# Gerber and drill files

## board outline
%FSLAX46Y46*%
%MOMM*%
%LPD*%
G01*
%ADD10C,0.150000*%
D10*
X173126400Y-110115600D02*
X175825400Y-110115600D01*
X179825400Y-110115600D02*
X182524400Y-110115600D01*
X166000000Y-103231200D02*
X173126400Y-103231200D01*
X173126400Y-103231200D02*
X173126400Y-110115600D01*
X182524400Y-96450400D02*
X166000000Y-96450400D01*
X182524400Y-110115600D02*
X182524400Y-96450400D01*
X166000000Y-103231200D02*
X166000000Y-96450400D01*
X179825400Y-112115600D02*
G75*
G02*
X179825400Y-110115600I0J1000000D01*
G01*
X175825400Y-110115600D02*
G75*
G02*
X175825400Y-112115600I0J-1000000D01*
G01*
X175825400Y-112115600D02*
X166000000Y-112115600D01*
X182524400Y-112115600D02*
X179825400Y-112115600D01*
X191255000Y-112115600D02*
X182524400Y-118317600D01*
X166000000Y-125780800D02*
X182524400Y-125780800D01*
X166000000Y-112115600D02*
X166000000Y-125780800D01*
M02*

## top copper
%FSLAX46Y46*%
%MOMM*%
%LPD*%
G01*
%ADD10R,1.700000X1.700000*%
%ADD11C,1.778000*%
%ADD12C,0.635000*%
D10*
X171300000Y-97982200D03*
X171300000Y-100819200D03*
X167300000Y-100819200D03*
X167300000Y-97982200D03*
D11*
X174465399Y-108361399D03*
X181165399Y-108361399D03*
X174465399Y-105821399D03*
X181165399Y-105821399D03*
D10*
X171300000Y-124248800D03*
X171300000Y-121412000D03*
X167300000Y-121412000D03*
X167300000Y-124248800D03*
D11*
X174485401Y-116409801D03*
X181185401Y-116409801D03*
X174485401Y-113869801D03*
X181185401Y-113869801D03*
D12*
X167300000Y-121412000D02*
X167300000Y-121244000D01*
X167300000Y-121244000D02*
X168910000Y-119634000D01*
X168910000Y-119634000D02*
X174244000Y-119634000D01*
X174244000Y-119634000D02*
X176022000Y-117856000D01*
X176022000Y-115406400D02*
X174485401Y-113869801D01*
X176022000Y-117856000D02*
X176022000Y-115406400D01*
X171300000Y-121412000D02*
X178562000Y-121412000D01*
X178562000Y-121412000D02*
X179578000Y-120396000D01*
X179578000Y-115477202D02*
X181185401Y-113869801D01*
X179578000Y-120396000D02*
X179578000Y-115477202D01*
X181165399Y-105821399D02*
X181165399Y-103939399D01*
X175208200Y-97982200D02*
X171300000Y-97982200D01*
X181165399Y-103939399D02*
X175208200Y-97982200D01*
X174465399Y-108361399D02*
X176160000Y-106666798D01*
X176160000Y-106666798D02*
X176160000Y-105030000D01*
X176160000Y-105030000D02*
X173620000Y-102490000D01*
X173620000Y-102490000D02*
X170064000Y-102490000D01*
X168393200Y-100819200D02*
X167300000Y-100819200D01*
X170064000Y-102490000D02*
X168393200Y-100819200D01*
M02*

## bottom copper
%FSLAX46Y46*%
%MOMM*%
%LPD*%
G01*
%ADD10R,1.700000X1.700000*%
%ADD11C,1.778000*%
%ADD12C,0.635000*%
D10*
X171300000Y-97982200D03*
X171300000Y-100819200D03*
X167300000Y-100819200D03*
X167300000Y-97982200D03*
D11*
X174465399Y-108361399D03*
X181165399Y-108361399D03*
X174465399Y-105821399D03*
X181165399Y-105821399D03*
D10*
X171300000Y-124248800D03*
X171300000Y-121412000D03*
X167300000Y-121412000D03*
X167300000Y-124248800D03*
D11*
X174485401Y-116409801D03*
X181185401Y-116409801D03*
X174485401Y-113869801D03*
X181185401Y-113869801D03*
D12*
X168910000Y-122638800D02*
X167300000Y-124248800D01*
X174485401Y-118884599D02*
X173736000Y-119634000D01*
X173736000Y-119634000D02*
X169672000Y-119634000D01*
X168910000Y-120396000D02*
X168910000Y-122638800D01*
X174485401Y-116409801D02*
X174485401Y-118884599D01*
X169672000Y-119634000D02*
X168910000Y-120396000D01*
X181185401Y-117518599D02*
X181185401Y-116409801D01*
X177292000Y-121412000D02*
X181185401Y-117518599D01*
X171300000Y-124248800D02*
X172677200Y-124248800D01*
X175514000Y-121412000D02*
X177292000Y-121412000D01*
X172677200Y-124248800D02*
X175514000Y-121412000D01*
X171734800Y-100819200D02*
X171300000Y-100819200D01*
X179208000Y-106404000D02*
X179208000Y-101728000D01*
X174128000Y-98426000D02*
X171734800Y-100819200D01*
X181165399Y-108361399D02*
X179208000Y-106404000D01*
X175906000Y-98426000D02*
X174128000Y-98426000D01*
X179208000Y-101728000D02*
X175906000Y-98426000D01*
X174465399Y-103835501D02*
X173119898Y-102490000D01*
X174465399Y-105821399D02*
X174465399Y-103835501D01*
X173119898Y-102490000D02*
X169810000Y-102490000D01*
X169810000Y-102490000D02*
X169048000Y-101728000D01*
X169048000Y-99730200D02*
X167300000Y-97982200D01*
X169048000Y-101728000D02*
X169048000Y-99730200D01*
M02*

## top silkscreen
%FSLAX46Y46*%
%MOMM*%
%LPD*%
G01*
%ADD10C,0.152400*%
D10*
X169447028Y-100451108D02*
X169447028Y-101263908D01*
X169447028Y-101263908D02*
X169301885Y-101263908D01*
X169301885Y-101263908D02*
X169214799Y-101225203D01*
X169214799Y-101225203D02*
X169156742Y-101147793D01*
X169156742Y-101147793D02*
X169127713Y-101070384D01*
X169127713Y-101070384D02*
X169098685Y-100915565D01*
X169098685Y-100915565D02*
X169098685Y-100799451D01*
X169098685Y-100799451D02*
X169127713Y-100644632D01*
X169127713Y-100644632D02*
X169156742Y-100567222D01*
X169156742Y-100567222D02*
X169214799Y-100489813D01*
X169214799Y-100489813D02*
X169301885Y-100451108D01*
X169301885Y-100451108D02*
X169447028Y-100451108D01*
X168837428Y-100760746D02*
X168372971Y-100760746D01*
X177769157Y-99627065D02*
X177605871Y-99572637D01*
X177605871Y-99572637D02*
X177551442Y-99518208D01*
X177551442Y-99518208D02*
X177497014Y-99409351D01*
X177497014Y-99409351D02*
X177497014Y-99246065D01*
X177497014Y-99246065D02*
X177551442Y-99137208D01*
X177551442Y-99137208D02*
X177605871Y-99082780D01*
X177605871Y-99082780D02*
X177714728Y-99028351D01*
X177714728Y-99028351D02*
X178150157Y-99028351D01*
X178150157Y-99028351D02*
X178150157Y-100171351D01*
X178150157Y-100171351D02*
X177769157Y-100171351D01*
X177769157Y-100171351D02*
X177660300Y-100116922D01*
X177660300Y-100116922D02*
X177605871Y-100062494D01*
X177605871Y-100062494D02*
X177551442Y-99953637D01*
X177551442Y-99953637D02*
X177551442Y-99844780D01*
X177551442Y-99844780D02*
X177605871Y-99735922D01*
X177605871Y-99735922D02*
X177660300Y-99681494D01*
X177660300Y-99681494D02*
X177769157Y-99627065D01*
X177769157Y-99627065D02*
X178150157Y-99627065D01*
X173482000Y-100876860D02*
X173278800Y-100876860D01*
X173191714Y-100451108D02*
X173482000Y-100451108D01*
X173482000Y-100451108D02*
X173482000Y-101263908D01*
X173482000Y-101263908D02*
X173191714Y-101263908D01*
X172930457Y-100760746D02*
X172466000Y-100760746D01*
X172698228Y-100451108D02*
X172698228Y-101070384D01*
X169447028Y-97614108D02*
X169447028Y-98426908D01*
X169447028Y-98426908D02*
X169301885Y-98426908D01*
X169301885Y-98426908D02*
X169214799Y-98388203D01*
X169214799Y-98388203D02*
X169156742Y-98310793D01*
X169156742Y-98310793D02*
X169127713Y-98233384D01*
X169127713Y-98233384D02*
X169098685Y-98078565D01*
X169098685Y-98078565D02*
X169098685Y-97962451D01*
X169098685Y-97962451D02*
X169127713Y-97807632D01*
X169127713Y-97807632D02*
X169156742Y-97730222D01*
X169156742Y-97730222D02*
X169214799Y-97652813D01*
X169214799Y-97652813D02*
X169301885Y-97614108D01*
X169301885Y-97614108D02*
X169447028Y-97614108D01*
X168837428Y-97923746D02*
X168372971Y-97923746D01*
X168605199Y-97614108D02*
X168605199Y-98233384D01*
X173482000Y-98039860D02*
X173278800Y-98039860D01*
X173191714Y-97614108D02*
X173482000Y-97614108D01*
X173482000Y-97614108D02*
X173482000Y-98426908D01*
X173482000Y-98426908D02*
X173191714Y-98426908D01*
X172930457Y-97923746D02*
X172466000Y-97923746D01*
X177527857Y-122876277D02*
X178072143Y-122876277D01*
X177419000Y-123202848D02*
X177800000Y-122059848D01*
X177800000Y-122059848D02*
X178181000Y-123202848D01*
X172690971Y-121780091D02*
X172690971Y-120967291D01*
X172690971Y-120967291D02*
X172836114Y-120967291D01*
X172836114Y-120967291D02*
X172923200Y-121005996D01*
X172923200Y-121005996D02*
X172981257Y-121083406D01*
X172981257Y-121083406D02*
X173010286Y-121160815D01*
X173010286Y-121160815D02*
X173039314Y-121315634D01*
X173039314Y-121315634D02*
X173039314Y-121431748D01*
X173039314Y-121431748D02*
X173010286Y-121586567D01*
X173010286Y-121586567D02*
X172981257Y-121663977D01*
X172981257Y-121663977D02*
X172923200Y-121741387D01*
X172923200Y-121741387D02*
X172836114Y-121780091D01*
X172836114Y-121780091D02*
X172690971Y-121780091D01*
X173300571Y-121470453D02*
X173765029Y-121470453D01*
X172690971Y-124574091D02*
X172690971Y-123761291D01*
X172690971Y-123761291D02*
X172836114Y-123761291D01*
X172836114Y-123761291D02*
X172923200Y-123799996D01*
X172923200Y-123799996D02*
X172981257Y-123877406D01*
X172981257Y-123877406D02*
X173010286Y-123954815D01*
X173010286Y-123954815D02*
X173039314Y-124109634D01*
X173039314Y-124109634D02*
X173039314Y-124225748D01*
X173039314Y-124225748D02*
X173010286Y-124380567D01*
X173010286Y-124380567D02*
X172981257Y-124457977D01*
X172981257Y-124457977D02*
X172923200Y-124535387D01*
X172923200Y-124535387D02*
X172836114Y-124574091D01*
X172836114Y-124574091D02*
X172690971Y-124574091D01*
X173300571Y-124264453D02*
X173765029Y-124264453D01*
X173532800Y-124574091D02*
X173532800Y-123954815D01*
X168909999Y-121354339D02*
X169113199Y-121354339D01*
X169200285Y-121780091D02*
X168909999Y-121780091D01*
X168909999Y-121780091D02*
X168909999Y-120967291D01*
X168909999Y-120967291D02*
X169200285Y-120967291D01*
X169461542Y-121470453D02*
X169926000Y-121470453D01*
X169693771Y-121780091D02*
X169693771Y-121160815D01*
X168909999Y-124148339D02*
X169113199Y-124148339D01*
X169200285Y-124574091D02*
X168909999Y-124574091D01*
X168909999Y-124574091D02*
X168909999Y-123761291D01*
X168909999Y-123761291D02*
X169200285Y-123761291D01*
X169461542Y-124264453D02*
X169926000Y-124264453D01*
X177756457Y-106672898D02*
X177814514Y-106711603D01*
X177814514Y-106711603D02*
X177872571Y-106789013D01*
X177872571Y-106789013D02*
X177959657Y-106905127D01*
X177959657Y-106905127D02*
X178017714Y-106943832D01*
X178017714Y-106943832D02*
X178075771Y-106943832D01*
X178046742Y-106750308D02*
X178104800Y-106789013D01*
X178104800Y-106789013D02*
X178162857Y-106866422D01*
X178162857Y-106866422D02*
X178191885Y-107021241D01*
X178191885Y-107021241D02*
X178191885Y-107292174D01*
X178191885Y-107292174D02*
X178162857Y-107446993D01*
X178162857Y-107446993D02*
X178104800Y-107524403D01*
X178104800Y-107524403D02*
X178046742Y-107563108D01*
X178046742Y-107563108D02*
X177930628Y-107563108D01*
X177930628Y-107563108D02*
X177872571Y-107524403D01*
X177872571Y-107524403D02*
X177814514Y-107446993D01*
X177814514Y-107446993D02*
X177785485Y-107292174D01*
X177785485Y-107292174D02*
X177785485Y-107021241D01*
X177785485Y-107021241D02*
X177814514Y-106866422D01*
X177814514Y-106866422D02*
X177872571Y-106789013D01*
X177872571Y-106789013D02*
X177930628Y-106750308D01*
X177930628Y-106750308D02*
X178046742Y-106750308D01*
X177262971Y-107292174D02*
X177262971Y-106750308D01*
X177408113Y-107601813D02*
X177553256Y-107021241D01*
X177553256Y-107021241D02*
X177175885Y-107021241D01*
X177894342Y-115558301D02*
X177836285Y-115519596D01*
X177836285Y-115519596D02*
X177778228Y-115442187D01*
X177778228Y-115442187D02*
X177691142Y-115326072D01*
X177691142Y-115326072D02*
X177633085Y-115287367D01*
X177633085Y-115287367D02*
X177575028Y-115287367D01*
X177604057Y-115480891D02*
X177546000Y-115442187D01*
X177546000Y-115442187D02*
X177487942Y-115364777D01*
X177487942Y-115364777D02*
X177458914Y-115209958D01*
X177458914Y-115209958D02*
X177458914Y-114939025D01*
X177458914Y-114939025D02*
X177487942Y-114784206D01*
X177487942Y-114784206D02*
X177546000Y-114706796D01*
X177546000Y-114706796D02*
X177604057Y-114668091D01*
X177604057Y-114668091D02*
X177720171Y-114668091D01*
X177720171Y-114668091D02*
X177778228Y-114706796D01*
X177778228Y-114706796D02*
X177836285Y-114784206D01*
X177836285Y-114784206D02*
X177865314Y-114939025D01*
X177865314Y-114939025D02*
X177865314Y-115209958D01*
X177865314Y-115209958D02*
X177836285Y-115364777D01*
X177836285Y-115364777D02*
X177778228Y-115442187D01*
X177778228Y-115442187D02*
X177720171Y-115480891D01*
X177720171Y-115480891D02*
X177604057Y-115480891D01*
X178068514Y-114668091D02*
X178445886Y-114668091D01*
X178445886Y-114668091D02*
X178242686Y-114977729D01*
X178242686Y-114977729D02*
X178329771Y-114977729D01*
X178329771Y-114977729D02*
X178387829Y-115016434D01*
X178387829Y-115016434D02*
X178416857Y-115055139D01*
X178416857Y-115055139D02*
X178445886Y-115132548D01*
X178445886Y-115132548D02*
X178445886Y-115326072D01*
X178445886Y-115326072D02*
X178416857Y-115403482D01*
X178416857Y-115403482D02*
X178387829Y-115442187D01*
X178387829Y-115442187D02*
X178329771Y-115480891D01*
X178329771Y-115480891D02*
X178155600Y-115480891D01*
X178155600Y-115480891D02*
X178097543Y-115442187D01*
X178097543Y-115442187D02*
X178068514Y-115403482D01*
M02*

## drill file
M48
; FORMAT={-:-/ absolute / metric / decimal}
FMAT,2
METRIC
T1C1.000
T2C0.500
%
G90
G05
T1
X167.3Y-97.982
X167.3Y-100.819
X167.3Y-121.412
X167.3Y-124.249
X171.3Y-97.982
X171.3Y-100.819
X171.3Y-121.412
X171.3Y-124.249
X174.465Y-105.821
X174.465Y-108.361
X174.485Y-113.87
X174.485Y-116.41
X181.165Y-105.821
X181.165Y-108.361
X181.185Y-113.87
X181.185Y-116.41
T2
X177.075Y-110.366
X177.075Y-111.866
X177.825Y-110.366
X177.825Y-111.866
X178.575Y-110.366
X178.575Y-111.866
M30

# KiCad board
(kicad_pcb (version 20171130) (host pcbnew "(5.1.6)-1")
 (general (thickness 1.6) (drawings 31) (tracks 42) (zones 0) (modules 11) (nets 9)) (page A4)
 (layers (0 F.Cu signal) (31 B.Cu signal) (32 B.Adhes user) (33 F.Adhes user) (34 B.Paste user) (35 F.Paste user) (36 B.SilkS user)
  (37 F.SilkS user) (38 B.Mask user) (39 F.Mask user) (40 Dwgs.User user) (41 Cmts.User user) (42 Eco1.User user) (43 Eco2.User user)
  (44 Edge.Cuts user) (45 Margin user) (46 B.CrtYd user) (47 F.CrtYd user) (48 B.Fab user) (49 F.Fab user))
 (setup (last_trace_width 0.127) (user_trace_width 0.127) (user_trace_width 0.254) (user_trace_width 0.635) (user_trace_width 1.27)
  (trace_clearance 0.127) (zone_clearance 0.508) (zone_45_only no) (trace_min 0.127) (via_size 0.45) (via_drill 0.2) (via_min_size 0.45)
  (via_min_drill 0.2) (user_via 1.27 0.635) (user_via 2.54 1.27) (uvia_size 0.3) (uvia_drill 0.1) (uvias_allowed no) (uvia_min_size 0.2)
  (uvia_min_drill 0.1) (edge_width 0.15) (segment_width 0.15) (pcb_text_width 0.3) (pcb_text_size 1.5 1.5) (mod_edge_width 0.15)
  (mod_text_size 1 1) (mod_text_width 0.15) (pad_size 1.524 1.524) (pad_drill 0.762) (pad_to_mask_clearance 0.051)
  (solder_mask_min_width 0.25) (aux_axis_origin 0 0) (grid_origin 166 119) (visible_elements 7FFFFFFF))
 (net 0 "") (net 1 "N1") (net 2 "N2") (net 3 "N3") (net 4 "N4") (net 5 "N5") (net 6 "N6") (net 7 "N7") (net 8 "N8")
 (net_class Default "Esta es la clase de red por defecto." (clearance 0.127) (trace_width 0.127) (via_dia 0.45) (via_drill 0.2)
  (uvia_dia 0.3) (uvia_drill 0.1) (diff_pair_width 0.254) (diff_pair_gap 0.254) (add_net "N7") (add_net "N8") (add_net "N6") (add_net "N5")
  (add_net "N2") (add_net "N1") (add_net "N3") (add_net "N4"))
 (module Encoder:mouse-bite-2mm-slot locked (layer F.Cu) (at 177.8254 111.1156)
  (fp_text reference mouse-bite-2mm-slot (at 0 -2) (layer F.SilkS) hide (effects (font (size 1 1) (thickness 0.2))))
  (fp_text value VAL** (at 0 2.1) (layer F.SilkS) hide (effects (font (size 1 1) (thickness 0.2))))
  (pad "" np_thru_hole circle (at 0.75 0.75) (size 0.5 0.5) (drill 0.5) (layers *.Cu *.Mask))
  (pad "" np_thru_hole circle (at -0.75 0.75) (size 0.5 0.5) (drill 0.5) (layers *.Cu *.Mask))
  (pad "" np_thru_hole circle (at -0.75 -0.75) (size 0.5 0.5) (drill 0.5) (layers *.Cu *.Mask))
  (pad "" np_thru_hole circle (at 0.75 -0.75) (size 0.5 0.5) (drill 0.5) (layers *.Cu *.Mask))
  (pad "" np_thru_hole circle (at 0 0.75) (size 0.5 0.5) (drill 0.5) (layers *.Cu *.Mask))
  (pad "" np_thru_hole circle (at 0 -0.75) (size 0.5 0.5) (drill 0.5) (layers *.Cu *.Mask)))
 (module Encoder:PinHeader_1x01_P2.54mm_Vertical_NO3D (layer F.Cu) (at 171.3 97.9822 180)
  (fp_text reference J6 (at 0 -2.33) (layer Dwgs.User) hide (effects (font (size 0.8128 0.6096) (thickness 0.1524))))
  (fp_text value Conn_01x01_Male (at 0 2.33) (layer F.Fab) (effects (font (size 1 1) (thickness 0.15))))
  (pad 1 thru_hole rect (at 0 0 180) (size 1.7 1.7) (drill 1) (layers *.Cu *.Mask) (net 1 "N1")))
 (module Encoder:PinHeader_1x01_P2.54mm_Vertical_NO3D (layer F.Cu) (at 171.3 100.8192 180)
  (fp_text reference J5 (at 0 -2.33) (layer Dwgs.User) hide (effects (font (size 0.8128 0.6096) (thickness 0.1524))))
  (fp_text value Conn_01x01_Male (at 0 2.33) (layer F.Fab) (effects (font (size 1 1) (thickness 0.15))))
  (pad 1 thru_hole rect (at 0 0 180) (size 1.7 1.7) (drill 1) (layers *.Cu *.Mask) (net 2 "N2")))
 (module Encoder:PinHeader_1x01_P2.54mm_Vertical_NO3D (layer F.Cu) (at 167.3 100.8192 180)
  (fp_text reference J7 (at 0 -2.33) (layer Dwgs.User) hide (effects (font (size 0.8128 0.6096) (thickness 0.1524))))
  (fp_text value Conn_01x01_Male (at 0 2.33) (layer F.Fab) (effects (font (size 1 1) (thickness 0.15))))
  (pad 1 thru_hole rect (at 0 0 180) (size 1.7 1.7) (drill 1) (layers *.Cu *.Mask) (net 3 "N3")))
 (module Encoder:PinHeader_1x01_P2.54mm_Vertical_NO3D (layer F.Cu) (at 167.3 97.9822 180)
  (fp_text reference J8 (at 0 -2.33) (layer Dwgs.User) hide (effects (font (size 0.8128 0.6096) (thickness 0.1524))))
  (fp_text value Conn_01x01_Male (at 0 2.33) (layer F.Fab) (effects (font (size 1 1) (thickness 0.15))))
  (pad 1 thru_hole rect (at 0 0 180) (size 1.7 1.7) (drill 1) (layers *.Cu *.Mask) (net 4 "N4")))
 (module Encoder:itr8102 (layer F.Cu) (at 177.815399 107.091399 180)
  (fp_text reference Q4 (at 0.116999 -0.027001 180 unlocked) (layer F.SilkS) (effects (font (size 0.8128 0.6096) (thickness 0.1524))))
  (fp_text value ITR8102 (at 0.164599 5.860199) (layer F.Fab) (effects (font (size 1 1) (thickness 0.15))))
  (pad 4 thru_hole circle (at 3.35 -1.27 180) (size 1.778 1.778) (drill 1) (layers *.Cu *.Mask) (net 3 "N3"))
  (pad 1 thru_hole circle (at -3.35 -1.27 180) (size 1.778 1.778) (drill 1) (layers *.Cu *.Mask) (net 2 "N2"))
  (pad 3 thru_hole circle (at 3.35 1.27 180) (size 1.778 1.778) (drill 1) (layers *.Cu *.Mask) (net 4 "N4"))
  (pad 2 thru_hole circle (at -3.35 1.27 180) (size 1.778 1.778) (drill 1) (layers *.Cu *.Mask) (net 1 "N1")))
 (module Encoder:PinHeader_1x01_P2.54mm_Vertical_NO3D (layer F.Cu) (at 171.3 124.2488)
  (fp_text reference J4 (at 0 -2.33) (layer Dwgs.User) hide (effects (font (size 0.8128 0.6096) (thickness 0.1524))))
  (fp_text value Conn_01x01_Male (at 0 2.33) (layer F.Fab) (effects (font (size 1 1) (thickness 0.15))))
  (pad 1 thru_hole rect (at 0 0) (size 1.7 1.7) (drill 1) (layers *.Cu *.Mask) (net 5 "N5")))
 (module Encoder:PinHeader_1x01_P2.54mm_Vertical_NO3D (layer F.Cu) (at 171.3 121.412)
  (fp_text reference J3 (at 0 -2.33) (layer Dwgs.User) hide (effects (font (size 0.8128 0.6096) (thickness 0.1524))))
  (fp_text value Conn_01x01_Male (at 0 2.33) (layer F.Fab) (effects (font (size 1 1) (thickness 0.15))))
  (pad 1 thru_hole rect (at 0 0) (size 1.7 1.7) (drill 1) (layers *.Cu *.Mask) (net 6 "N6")))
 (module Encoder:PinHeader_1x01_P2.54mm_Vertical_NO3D (layer F.Cu) (at 167.3 121.412)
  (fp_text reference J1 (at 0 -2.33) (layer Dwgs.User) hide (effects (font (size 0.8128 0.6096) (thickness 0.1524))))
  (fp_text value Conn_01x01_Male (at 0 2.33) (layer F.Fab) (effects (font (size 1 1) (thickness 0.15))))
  (pad 1 thru_hole rect (at 0 0) (size 1.7 1.7) (drill 1) (layers *.Cu *.Mask) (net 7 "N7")))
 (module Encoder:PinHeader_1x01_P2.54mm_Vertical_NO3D (layer F.Cu) (at 167.3 124.2488)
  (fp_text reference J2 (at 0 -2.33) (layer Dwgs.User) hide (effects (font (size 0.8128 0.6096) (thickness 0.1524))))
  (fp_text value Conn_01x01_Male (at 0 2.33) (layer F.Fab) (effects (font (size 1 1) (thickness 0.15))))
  (pad 1 thru_hole rect (at 0 0) (size 1.7 1.7) (drill 1) (layers *.Cu *.Mask) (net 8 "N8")))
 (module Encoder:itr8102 (layer F.Cu) (at 177.835401 115.139801)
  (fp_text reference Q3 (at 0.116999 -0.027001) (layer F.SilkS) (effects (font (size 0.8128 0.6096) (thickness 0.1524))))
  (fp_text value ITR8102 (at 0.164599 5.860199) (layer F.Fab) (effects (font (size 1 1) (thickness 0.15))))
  (pad 2 thru_hole circle (at -3.35 1.27) (size 1.778 1.778) (drill 1) (layers *.Cu *.Mask) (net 8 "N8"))
  (pad 3 thru_hole circle (at 3.35 1.27) (size 1.778 1.778) (drill 1) (layers *.Cu *.Mask) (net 5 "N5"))
  (pad 1 thru_hole circle (at -3.35 -1.27) (size 1.778 1.778) (drill 1) (layers *.Cu *.Mask) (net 7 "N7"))
  (pad 4 thru_hole circle (at 3.35 -1.27) (size 1.778 1.778) (drill 1) (layers *.Cu *.Mask) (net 6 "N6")))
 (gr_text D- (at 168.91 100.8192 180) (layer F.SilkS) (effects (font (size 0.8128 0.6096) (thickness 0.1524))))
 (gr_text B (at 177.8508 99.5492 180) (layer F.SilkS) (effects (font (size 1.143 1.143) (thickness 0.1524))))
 (gr_line (start 173.1264 110.1156) (end 175.8254 110.1156) (layer Edge.Cuts) (width 0.15))
 (gr_line (start 179.8254 110.1156) (end 182.5244 110.1156) (layer Edge.Cuts) (width 0.15))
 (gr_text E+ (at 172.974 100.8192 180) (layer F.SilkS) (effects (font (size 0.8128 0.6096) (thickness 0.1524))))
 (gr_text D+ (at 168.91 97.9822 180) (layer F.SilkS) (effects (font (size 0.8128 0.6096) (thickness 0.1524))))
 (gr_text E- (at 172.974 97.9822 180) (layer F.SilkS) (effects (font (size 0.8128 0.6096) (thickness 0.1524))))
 (gr_line (start 166 103.2312) (end 173.1264 103.2312) (layer Edge.Cuts) (width 0.15))
 (gr_line (start 173.1264 103.2312) (end 173.1264 110.1156) (layer Edge.Cuts) (width 0.15))
 (gr_line (start 182.5244 96.4504) (end 166 96.4504) (layer Edge.Cuts) (width 0.15))
 (gr_line (start 182.5244 110.1156) (end 182.5244 96.4504) (layer Edge.Cuts) (width 0.15))
 (gr_line (start 166 103.2312) (end 166 96.4504) (layer Edge.Cuts) (width 0.15))
 (gr_arc (start 179.8254 111.1156) (end 179.8254 110.1156) (angle -180) (layer Edge.Cuts) (width 0.15))
 (gr_arc (start 175.8254 111.1156) (end 175.8254 112.1156) (angle -180) (layer Edge.Cuts) (width 0.15))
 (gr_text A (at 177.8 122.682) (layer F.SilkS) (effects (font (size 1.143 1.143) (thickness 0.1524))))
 (gr_line (start 175.8254 112.1156) (end 166 112.1156) (layer Edge.Cuts) (width 0.15))
 (gr_line (start 182.5244 112.1156) (end 179.8254 112.1156) (layer Edge.Cuts) (width 0.15))
 (gr_line (start 191.255 112.1156) (end 182.5244 118.3176) (layer Edge.Cuts) (width 0.15))
 (gr_line (start 166 125.7808) (end 182.5244 125.7808) (layer Edge.Cuts) (width 0.15))
 (gr_line (start 166 112.1156) (end 166 125.7808) (layer Edge.Cuts) (width 0.15))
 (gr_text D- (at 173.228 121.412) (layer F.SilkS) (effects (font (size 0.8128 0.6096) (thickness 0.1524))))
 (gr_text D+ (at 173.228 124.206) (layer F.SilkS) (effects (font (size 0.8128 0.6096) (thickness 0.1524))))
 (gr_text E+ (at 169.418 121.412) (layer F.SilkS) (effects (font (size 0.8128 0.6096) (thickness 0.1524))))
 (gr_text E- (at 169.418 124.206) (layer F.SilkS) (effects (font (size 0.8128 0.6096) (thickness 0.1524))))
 (segment (start 167.3 121.412) (end 167.3 121.244) (width 0.635) (layer F.Cu) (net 7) (status 30))
 (segment (start 167.3 121.244) (end 168.91 119.634) (width 0.635) (layer F.Cu) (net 7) (status 10))
 (segment (start 168.91 119.634) (end 174.244 119.634) (width 0.635) (layer F.Cu) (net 7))
 (segment (start 174.244 119.634) (end 176.022 117.856) (width 0.635) (layer F.Cu) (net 7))
 (segment (start 176.022 115.4064) (end 174.485401 113.869801) (width 0.635) (layer F.Cu) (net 7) (status 20))
 (segment (start 176.022 117.856) (end 176.022 115.4064) (width 0.635) (layer F.Cu) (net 7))
 (segment (start 168.91 122.6388) (end 167.3 124.2488) (width 0.635) (layer B.Cu) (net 8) (status 20))
 (segment (start 174.485401 118.884599) (end 173.736 119.634) (width 0.635) (layer B.Cu) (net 8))
 (segment (start 173.736 119.634) (end 169.672 119.634) (width 0.635) (layer B.Cu) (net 8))
 (segment (start 168.91 120.396) (end 168.91 122.6388) (width 0.635) (layer B.Cu) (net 8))
 (segment (start 174.485401 116.409801) (end 174.485401 118.884599) (width 0.635) (layer B.Cu) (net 8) (status 10))
 (segment (start 169.672 119.634) (end 168.91 120.396) (width 0.635) (layer B.Cu) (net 8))
 (segment (start 171.3 121.412) (end 178.562 121.412) (width 0.635) (layer F.Cu) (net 6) (status 10))
 (segment (start 178.562 121.412) (end 179.578 120.396) (width 0.635) (layer F.Cu) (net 6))
 (segment (start 179.578 115.477202) (end 181.185401 113.869801) (width 0.635) (layer F.Cu) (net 6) (status 20))
 (segment (start 179.578 120.396) (end 179.578 115.477202) (width 0.635) (layer F.Cu) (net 6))
 (segment (start 181.185401 117.518599) (end 181.185401 116.409801) (width 0.635) (layer B.Cu) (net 5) (status 20))
 (segment (start 177.292 121.412) (end 181.185401 117.518599) (width 0.635) (layer B.Cu) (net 5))
 (segment (start 171.3 124.2488) (end 172.6772 124.2488) (width 0.635) (layer B.Cu) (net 5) (status 10))
 (segment (start 175.514 121.412) (end 177.292 121.412) (width 0.635) (layer B.Cu) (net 5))
 (segment (start 172.6772 124.2488) (end 175.514 121.412) (width 0.635) (layer B.Cu) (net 5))
 (segment (start 171.7348 100.8192) (end 171.3 100.8192) (width 0.635) (layer B.Cu) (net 2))
 (segment (start 179.208 106.404) (end 179.208 101.728) (width 0.635) (layer B.Cu) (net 2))
 (segment (start 174.128 98.426) (end 171.7348 100.8192) (width 0.635) (layer B.Cu) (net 2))
 (segment (start 181.165399 108.361399) (end 179.208 106.404) (width 0.635) (layer B.Cu) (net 2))
 (segment (start 175.906 98.426) (end 174.128 98.426) (width 0.635) (layer B.Cu) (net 2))
 (segment (start 179.208 101.728) (end 175.906 98.426) (width 0.635) (layer B.Cu) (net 2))
 (segment (start 181.165399 105.821399) (end 181.165399 103.939399) (width 0.635) (layer F.Cu) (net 1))
 (segment (start 175.2082 97.9822) (end 171.3 97.9822) (width 0.635) (layer F.Cu) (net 1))
 (segment (start 181.165399 103.939399) (end 175.2082 97.9822) (width 0.635) (layer F.Cu) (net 1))
 (segment (start 174.465399 108.361399) (end 176.16 106.666798) (width 0.635) (layer F.Cu) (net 3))
 (segment (start 176.16 106.666798) (end 176.16 105.03) (width 0.635) (layer F.Cu) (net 3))
 (segment (start 176.16 105.03) (end 173.62 102.49) (width 0.635) (layer F.Cu) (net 3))
 (segment (start 173.62 102.49) (end 170.064 102.49) (width 0.635) (layer F.Cu) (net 3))
 (segment (start 168.3932 100.8192) (end 167.3 100.8192) (width 0.635) (layer F.Cu) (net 3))
 (segment (start 170.064 102.49) (end 168.3932 100.8192) (width 0.635) (layer F.Cu) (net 3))
 (segment (start 174.465399 103.835501) (end 173.119898 102.49) (width 0.635) (layer B.Cu) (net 4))
 (segment (start 174.465399 105.821399) (end 174.465399 103.835501) (width 0.635) (layer B.Cu) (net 4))
 (segment (start 173.119898 102.49) (end 169.81 102.49) (width 0.635) (layer B.Cu) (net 4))
 (segment (start 169.81 102.49) (end 169.048 101.728) (width 0.635) (layer B.Cu) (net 4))
 (segment (start 169.048 99.7302) (end 167.3 97.9822) (width 0.635) (layer B.Cu) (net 4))
 (segment (start 169.048 101.728) (end 169.048 99.7302) (width 0.635) (layer B.Cu) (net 4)))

